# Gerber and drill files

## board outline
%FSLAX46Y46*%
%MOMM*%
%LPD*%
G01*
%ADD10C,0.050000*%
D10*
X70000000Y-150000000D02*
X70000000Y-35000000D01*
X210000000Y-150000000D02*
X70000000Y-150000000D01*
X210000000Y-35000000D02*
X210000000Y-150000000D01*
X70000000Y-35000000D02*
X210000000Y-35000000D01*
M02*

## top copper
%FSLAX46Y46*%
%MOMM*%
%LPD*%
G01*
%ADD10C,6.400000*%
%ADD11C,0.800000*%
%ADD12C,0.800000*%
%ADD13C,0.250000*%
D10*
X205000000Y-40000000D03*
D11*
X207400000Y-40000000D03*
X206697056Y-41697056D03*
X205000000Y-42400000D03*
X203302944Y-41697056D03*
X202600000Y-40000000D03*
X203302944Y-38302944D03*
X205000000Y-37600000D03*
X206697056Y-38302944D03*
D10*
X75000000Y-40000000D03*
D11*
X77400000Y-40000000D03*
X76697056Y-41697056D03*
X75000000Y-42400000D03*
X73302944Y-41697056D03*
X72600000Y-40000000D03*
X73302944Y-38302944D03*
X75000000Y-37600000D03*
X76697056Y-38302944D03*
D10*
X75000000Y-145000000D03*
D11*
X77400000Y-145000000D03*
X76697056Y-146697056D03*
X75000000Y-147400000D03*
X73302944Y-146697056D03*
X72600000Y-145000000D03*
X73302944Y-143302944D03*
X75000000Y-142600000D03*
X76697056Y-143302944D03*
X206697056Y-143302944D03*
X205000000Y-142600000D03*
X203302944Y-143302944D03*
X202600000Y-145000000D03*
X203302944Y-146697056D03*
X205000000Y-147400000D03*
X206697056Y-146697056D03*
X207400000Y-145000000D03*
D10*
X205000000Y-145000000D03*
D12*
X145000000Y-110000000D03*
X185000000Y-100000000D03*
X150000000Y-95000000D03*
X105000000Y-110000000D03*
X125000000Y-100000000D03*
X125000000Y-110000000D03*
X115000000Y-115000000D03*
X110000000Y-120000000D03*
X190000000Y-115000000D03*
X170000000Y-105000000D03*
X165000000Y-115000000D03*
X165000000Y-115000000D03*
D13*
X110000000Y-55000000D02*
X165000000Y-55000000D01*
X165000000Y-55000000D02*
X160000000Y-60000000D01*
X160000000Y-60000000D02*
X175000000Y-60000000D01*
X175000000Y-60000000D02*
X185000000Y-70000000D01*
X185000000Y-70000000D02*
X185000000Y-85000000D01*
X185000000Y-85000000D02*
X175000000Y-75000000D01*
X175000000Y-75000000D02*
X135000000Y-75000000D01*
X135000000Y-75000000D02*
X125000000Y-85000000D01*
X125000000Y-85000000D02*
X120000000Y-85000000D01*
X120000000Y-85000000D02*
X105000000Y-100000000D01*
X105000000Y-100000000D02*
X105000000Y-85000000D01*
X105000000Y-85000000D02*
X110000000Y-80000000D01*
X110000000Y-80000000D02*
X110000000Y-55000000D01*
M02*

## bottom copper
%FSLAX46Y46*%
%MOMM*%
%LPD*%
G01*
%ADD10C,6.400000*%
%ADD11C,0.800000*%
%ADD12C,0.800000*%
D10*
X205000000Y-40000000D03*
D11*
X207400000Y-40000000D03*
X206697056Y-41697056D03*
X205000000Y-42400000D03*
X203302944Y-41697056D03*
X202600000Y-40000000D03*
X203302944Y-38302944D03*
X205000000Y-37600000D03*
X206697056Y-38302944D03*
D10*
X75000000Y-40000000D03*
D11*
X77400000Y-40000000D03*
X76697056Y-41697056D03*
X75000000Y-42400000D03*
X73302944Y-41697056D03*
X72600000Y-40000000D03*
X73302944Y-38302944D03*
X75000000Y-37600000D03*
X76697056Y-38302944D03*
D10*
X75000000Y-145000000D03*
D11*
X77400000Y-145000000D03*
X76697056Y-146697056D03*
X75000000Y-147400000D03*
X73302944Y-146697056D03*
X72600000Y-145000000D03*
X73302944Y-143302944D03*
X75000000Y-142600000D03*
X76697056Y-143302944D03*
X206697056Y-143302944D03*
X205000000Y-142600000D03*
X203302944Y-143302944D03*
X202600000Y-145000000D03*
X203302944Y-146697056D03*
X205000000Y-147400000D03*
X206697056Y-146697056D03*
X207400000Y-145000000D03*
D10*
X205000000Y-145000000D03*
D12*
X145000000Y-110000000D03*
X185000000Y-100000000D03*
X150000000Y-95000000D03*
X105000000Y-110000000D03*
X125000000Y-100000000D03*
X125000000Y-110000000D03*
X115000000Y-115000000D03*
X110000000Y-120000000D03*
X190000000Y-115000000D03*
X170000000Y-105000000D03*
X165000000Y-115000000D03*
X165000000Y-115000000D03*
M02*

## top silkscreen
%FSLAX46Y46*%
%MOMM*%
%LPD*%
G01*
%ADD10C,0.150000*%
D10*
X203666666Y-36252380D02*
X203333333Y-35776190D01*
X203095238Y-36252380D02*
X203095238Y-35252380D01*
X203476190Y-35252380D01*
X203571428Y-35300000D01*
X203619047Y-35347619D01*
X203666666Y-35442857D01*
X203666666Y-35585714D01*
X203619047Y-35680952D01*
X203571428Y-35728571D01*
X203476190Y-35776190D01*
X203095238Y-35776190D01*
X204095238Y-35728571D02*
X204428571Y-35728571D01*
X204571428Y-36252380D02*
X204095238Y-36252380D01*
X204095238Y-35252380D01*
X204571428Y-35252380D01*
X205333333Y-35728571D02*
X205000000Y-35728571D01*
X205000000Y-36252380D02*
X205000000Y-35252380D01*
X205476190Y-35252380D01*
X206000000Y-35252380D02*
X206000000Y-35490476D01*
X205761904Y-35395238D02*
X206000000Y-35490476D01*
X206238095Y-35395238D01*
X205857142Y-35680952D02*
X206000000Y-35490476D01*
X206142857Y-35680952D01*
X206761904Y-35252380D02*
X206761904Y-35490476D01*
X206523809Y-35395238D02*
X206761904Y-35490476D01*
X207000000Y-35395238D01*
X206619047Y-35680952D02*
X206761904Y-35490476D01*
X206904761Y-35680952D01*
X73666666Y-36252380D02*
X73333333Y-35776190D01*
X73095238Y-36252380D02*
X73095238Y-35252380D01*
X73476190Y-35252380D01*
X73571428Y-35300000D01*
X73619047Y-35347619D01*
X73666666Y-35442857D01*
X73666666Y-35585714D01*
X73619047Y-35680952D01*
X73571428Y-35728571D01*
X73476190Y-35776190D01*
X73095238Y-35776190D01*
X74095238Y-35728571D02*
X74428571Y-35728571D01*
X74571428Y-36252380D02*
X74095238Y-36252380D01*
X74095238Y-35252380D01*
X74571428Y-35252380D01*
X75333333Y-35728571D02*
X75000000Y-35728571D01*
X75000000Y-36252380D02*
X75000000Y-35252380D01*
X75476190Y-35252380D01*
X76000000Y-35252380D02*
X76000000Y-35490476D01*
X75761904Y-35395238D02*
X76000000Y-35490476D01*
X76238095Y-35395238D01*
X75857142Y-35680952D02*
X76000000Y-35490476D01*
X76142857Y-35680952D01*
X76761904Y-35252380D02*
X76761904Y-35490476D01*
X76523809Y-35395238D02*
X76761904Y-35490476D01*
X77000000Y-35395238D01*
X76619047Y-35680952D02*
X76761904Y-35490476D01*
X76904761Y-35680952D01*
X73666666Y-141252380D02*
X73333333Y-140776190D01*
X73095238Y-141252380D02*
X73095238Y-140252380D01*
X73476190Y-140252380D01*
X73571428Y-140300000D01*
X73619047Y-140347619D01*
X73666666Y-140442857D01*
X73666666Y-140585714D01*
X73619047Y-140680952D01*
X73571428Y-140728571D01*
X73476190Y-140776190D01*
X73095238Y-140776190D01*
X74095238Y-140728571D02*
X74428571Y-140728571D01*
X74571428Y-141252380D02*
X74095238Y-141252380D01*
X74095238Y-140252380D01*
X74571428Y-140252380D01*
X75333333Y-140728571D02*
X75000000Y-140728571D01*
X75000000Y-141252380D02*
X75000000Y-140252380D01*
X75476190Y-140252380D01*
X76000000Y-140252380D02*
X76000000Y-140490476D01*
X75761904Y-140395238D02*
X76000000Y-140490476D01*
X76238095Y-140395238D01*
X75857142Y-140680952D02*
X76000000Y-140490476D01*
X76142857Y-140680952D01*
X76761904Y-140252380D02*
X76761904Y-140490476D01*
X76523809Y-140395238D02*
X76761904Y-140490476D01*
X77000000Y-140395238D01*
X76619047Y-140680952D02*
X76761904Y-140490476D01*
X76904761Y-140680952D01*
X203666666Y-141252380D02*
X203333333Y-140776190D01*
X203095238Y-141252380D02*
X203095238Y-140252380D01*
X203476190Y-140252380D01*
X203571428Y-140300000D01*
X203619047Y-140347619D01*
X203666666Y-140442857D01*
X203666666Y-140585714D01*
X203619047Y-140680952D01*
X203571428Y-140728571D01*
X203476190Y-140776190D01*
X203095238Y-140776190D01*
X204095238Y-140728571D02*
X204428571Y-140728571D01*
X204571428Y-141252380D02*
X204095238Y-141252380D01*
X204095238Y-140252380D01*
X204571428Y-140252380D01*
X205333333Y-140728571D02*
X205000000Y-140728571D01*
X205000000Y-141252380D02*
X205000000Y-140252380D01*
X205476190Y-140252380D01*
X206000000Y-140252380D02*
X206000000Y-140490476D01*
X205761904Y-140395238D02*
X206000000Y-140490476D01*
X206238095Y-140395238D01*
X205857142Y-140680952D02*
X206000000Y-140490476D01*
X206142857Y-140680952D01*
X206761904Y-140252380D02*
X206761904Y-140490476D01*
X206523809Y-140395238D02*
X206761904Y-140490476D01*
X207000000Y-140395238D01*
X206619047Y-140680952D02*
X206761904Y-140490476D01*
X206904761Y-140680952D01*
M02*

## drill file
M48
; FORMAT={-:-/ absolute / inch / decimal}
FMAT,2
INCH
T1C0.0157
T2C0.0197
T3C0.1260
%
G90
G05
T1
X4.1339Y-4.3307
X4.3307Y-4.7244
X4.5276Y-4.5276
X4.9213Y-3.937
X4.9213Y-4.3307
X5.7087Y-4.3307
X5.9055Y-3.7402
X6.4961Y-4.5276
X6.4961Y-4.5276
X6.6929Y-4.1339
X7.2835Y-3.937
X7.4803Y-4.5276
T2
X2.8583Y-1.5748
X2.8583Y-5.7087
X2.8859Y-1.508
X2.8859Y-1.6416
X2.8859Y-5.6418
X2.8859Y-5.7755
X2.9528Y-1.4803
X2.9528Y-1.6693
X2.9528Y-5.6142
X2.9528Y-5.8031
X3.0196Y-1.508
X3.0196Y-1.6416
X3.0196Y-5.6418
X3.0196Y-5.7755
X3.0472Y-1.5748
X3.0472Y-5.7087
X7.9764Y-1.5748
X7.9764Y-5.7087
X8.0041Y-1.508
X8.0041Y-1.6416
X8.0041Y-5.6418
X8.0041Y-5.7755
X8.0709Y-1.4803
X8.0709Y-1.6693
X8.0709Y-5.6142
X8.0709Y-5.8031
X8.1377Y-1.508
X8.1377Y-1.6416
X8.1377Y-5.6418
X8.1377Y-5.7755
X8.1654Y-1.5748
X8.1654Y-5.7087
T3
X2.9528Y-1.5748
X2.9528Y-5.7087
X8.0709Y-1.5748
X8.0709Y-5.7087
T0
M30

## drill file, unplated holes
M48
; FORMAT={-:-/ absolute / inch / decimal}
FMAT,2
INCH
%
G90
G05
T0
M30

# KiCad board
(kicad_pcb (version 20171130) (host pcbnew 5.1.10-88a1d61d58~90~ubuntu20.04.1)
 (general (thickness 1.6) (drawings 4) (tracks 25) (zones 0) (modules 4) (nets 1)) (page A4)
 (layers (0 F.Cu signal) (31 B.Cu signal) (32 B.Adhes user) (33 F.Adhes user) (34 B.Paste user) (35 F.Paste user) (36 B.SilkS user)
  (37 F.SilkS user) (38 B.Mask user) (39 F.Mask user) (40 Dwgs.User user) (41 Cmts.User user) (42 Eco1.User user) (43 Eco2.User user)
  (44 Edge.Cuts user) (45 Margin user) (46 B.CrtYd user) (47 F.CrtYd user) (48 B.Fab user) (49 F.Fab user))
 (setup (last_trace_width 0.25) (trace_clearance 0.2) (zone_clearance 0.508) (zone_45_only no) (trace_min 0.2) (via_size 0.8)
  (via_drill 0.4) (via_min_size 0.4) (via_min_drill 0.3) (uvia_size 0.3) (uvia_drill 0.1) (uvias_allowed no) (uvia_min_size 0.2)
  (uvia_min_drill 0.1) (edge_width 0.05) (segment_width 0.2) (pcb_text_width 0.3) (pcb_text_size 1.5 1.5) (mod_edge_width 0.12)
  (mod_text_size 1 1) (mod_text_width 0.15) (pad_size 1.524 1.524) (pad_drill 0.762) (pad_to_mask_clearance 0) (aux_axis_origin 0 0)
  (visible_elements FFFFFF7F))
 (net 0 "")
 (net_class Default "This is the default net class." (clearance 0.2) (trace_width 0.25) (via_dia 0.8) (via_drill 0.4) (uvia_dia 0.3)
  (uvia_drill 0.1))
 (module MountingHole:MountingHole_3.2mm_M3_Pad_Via (layer F.Cu) (at 205 40)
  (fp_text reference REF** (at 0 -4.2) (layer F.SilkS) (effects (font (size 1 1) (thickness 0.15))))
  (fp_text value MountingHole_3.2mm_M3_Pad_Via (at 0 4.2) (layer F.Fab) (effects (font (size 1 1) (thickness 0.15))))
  (pad 1 thru_hole circle (at 0 0) (size 6.4 6.4) (drill 3.2) (layers *.Cu *.Mask))
  (pad 1 thru_hole circle (at 2.4 0) (size 0.8 0.8) (drill 0.5) (layers *.Cu *.Mask))
  (pad 1 thru_hole circle (at 1.697056 1.697056) (size 0.8 0.8) (drill 0.5) (layers *.Cu *.Mask))
  (pad 1 thru_hole circle (at 0 2.4) (size 0.8 0.8) (drill 0.5) (layers *.Cu *.Mask))
  (pad 1 thru_hole circle (at -1.697056 1.697056) (size 0.8 0.8) (drill 0.5) (layers *.Cu *.Mask))
  (pad 1 thru_hole circle (at -2.4 0) (size 0.8 0.8) (drill 0.5) (layers *.Cu *.Mask))
  (pad 1 thru_hole circle (at -1.697056 -1.697056) (size 0.8 0.8) (drill 0.5) (layers *.Cu *.Mask))
  (pad 1 thru_hole circle (at 0 -2.4) (size 0.8 0.8) (drill 0.5) (layers *.Cu *.Mask))
  (pad 1 thru_hole circle (at 1.697056 -1.697056) (size 0.8 0.8) (drill 0.5) (layers *.Cu *.Mask)))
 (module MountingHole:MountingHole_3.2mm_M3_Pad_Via (layer F.Cu) (at 75 40)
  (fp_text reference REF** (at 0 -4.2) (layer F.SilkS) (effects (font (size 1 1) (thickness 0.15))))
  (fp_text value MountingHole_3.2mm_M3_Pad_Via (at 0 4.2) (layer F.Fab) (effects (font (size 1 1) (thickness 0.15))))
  (pad 1 thru_hole circle (at 0 0) (size 6.4 6.4) (drill 3.2) (layers *.Cu *.Mask))
  (pad 1 thru_hole circle (at 2.4 0) (size 0.8 0.8) (drill 0.5) (layers *.Cu *.Mask))
  (pad 1 thru_hole circle (at 1.697056 1.697056) (size 0.8 0.8) (drill 0.5) (layers *.Cu *.Mask))
  (pad 1 thru_hole circle (at 0 2.4) (size 0.8 0.8) (drill 0.5) (layers *.Cu *.Mask))
  (pad 1 thru_hole circle (at -1.697056 1.697056) (size 0.8 0.8) (drill 0.5) (layers *.Cu *.Mask))
  (pad 1 thru_hole circle (at -2.4 0) (size 0.8 0.8) (drill 0.5) (layers *.Cu *.Mask))
  (pad 1 thru_hole circle (at -1.697056 -1.697056) (size 0.8 0.8) (drill 0.5) (layers *.Cu *.Mask))
  (pad 1 thru_hole circle (at 0 -2.4) (size 0.8 0.8) (drill 0.5) (layers *.Cu *.Mask))
  (pad 1 thru_hole circle (at 1.697056 -1.697056) (size 0.8 0.8) (drill 0.5) (layers *.Cu *.Mask)))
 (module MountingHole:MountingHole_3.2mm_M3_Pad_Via (layer F.Cu) (at 75 145)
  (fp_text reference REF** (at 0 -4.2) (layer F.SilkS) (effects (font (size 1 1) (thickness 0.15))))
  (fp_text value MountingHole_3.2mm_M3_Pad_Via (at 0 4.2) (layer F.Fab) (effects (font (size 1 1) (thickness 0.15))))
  (pad 1 thru_hole circle (at 0 0) (size 6.4 6.4) (drill 3.2) (layers *.Cu *.Mask))
  (pad 1 thru_hole circle (at 2.4 0) (size 0.8 0.8) (drill 0.5) (layers *.Cu *.Mask))
  (pad 1 thru_hole circle (at 1.697056 1.697056) (size 0.8 0.8) (drill 0.5) (layers *.Cu *.Mask))
  (pad 1 thru_hole circle (at 0 2.4) (size 0.8 0.8) (drill 0.5) (layers *.Cu *.Mask))
  (pad 1 thru_hole circle (at -1.697056 1.697056) (size 0.8 0.8) (drill 0.5) (layers *.Cu *.Mask))
  (pad 1 thru_hole circle (at -2.4 0) (size 0.8 0.8) (drill 0.5) (layers *.Cu *.Mask))
  (pad 1 thru_hole circle (at -1.697056 -1.697056) (size 0.8 0.8) (drill 0.5) (layers *.Cu *.Mask))
  (pad 1 thru_hole circle (at 0 -2.4) (size 0.8 0.8) (drill 0.5) (layers *.Cu *.Mask))
  (pad 1 thru_hole circle (at 1.697056 -1.697056) (size 0.8 0.8) (drill 0.5) (layers *.Cu *.Mask)))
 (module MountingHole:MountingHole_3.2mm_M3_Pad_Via (layer F.Cu) (at 205 145)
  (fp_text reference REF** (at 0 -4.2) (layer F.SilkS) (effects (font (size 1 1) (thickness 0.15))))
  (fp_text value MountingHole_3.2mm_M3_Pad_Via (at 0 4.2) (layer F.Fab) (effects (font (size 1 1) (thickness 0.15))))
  (pad 1 thru_hole circle (at 1.697056 -1.697056) (size 0.8 0.8) (drill 0.5) (layers *.Cu *.Mask))
  (pad 1 thru_hole circle (at 0 -2.4) (size 0.8 0.8) (drill 0.5) (layers *.Cu *.Mask))
  (pad 1 thru_hole circle (at -1.697056 -1.697056) (size 0.8 0.8) (drill 0.5) (layers *.Cu *.Mask))
  (pad 1 thru_hole circle (at -2.4 0) (size 0.8 0.8) (drill 0.5) (layers *.Cu *.Mask))
  (pad 1 thru_hole circle (at -1.697056 1.697056) (size 0.8 0.8) (drill 0.5) (layers *.Cu *.Mask))
  (pad 1 thru_hole circle (at 0 2.4) (size 0.8 0.8) (drill 0.5) (layers *.Cu *.Mask))
  (pad 1 thru_hole circle (at 1.697056 1.697056) (size 0.8 0.8) (drill 0.5) (layers *.Cu *.Mask))
  (pad 1 thru_hole circle (at 2.4 0) (size 0.8 0.8) (drill 0.5) (layers *.Cu *.Mask))
  (pad 1 thru_hole circle (at 0 0) (size 6.4 6.4) (drill 3.2) (layers *.Cu *.Mask)))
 (gr_line (start 70 150) (end 70 35) (layer Edge.Cuts) (width 0.05))
 (gr_line (start 210 150) (end 70 150) (layer Edge.Cuts) (width 0.05))
 (gr_line (start 210 35) (end 210 150) (layer Edge.Cuts) (width 0.05))
 (gr_line (start 70 35) (end 210 35) (layer Edge.Cuts) (width 0.05))
 (segment (start 110 55) (end 165 55) (width 0.25) (layer F.Cu) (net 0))
 (segment (start 165 55) (end 160 60) (width 0.25) (layer F.Cu) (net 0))
 (segment (start 160 60) (end 175 60) (width 0.25) (layer F.Cu) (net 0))
 (segment (start 175 60) (end 185 70) (width 0.25) (layer F.Cu) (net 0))
 (segment (start 185 70) (end 185 85) (width 0.25) (layer F.Cu) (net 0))
 (segment (start 185 85) (end 175 75) (width 0.25) (layer F.Cu) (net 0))
 (segment (start 175 75) (end 135 75) (width 0.25) (layer F.Cu) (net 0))
 (segment (start 135 75) (end 125 85) (width 0.25) (layer F.Cu) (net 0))
 (segment (start 125 85) (end 120 85) (width 0.25) (layer F.Cu) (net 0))
 (segment (start 120 85) (end 105 100) (width 0.25) (layer F.Cu) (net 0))
 (segment (start 105 100) (end 105 85) (width 0.25) (layer F.Cu) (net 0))
 (segment (start 105 85) (end 110 80) (width 0.25) (layer F.Cu) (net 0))
 (segment (start 110 80) (end 110 55) (width 0.25) (layer F.Cu) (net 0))
 (via (at 145 110) (size 0.8) (drill 0.4) (layers F.Cu B.Cu) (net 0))
 (via (at 185 100) (size 0.8) (drill 0.4) (layers F.Cu B.Cu) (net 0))
 (via (at 150 95) (size 0.8) (drill 0.4) (layers F.Cu B.Cu) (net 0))
 (via (at 105 110) (size 0.8) (drill 0.4) (layers F.Cu B.Cu) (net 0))
 (via (at 125 100) (size 0.8) (drill 0.4) (layers F.Cu B.Cu) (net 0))
 (via (at 125 110) (size 0.8) (drill 0.4) (layers F.Cu B.Cu) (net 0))
 (via (at 115 115) (size 0.8) (drill 0.4) (layers F.Cu B.Cu) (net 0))
 (via (at 110 120) (size 0.8) (drill 0.4) (layers F.Cu B.Cu) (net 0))
 (via (at 190 115) (size 0.8) (drill 0.4) (layers F.Cu B.Cu) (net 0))
 (via (at 170 105) (size 0.8) (drill 0.4) (layers F.Cu B.Cu) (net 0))
 (via (at 165 115) (size 0.8) (drill 0.4) (layers F.Cu B.Cu) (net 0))
 (via (at 165 115) (size 0.8) (drill 0.4) (layers F.Cu B.Cu) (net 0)))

